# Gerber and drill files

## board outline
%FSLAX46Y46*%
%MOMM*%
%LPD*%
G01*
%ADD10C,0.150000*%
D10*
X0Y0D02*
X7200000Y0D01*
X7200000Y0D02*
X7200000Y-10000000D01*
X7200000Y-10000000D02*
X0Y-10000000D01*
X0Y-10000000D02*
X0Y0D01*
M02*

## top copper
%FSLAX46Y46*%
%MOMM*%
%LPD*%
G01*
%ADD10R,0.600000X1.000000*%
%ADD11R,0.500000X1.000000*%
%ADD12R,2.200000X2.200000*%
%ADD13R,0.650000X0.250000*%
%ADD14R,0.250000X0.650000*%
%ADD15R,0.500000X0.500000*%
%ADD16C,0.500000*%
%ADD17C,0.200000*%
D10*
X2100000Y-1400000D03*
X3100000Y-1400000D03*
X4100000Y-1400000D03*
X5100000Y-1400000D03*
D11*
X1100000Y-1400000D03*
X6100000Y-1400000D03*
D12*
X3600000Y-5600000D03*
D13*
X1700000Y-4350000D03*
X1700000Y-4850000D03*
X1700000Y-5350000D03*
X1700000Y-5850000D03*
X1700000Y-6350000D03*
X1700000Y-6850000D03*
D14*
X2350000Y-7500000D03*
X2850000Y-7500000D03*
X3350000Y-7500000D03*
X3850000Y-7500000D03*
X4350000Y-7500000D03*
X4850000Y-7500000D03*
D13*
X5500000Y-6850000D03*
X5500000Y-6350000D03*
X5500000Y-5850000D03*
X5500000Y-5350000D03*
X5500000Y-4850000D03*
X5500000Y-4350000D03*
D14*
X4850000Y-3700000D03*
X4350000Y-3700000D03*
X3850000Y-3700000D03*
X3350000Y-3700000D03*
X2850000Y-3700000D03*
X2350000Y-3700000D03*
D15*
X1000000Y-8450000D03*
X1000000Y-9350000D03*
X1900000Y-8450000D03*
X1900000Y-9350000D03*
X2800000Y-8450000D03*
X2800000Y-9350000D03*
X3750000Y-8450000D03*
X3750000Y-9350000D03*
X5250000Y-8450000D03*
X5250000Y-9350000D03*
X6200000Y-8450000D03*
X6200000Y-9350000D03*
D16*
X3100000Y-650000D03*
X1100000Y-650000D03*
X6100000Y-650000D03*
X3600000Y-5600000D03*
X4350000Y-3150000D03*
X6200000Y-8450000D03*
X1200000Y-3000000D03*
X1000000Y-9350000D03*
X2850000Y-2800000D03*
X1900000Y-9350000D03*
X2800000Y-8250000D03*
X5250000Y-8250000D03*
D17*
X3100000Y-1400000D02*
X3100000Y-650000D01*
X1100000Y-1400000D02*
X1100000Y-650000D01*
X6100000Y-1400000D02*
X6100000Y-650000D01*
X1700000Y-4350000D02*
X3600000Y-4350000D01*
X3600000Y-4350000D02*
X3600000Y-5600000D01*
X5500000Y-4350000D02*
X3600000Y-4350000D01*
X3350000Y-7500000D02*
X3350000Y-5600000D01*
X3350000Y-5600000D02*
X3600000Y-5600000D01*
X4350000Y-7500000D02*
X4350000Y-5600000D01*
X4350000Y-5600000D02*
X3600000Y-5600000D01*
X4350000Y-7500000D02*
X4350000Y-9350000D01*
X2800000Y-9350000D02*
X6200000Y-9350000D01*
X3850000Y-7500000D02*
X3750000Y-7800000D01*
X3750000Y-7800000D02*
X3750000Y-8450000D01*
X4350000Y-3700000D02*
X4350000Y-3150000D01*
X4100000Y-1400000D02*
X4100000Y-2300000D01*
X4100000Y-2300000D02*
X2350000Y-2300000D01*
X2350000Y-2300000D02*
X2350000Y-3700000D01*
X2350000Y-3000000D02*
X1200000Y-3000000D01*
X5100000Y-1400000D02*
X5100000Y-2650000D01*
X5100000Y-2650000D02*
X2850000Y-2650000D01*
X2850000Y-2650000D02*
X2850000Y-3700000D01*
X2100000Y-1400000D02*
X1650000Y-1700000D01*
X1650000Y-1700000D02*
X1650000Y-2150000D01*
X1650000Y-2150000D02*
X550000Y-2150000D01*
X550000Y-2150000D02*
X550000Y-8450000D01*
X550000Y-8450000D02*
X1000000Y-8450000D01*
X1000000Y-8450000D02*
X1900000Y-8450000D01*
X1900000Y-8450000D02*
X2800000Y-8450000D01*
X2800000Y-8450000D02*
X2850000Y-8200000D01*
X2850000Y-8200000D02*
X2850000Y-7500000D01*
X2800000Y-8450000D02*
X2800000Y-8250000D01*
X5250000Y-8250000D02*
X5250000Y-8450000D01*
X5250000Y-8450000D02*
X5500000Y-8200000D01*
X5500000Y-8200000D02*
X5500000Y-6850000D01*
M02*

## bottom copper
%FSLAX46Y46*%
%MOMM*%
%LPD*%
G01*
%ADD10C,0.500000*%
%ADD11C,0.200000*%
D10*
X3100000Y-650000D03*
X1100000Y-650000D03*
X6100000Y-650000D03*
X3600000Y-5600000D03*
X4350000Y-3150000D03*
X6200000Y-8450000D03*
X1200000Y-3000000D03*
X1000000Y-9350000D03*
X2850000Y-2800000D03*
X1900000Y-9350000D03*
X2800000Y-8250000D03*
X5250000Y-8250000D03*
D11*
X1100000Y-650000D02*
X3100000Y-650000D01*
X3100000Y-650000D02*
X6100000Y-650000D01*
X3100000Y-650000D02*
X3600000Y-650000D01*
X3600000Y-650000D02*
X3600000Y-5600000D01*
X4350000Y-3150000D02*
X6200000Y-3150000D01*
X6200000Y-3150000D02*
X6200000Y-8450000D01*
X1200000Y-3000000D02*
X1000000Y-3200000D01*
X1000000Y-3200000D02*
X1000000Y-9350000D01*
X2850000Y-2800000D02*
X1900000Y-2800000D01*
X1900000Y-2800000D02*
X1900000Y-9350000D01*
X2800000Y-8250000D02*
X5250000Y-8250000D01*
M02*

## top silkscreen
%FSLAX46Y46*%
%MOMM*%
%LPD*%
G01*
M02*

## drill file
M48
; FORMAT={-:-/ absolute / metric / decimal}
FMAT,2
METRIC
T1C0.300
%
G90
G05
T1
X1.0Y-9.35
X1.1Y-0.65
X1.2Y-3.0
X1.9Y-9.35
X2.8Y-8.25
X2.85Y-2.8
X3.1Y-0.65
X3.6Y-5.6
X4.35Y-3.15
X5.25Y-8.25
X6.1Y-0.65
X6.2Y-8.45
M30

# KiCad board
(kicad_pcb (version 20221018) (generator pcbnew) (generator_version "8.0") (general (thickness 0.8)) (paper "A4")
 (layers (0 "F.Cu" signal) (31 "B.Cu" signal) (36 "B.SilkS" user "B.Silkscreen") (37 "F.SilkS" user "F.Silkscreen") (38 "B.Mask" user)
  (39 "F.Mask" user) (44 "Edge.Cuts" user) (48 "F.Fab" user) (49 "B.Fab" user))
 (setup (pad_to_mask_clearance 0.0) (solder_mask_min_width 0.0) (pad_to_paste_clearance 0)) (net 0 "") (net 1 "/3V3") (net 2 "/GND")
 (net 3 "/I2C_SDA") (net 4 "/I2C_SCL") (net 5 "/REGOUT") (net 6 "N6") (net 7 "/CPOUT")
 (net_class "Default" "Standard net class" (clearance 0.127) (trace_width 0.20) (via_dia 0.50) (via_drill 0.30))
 (gr_line (start 0 0) (end 7.2 0) (layer "Edge.Cuts") (width 0.15))
 (gr_line (start 7.2 0) (end 7.2 10.0) (layer "Edge.Cuts") (width 0.15))
 (gr_line (start 7.2 10.0) (end 0 10.0) (layer "Edge.Cuts") (width 0.15))
 (gr_line (start 0 10.0) (end 0 0) (layer "Edge.Cuts") (width 0.15))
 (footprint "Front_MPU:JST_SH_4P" (layer "F.Cu") (at 3.6 1.4)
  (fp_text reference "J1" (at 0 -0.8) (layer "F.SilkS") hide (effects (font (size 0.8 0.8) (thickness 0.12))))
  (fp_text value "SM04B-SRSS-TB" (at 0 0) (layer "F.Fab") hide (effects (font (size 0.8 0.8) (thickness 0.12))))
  (pad "1" smd rect (at -1.5 0) (size 0.6 1.0) (layers "F.Cu" "F.Paste" "F.Mask") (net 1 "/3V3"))
  (pad "2" smd rect (at -0.5 0) (size 0.6 1.0) (layers "F.Cu" "F.Paste" "F.Mask") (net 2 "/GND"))
  (pad "3" smd rect (at 0.5 0) (size 0.6 1.0) (layers "F.Cu" "F.Paste" "F.Mask") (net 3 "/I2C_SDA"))
  (pad "4" smd rect (at 1.5 0) (size 0.6 1.0) (layers "F.Cu" "F.Paste" "F.Mask") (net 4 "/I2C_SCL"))
  (pad "5" smd rect (at -2.5 0) (size 0.5 1.0) (layers "F.Cu" "F.Paste" "F.Mask") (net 2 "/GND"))
  (pad "5" smd rect (at 2.5 0) (size 0.5 1.0) (layers "F.Cu" "F.Paste" "F.Mask") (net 2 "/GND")))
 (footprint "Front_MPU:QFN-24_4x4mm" (layer "F.Cu") (at 3.6 5.6)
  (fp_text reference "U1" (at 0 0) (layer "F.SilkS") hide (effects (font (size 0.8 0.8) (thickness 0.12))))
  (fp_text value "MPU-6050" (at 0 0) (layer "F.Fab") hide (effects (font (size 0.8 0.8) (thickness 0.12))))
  (pad "25" smd rect (at 0 0) (size 2.2 2.2) (layers "F.Cu" "F.Paste" "F.Mask") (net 2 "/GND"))
  (pad "1" smd rect (at -1.90 -1.25) (size 0.65 0.25) (layers "F.Cu" "F.Paste" "F.Mask") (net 2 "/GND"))
  (pad "2" smd rect (at -1.90 -0.75) (size 0.65 0.25) (layers "F.Cu" "F.Paste" "F.Mask") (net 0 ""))
  (pad "3" smd rect (at -1.90 -0.25) (size 0.65 0.25) (layers "F.Cu" "F.Paste" "F.Mask") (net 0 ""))
  (pad "4" smd rect (at -1.90 0.25) (size 0.65 0.25) (layers "F.Cu" "F.Paste" "F.Mask") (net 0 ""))
  (pad "5" smd rect (at -1.90 0.75) (size 0.65 0.25) (layers "F.Cu" "F.Paste" "F.Mask") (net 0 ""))
  (pad "6" smd rect (at -1.90 1.25) (size 0.65 0.25) (layers "F.Cu" "F.Paste" "F.Mask") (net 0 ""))
  (pad "7" smd rect (at -1.25 1.90) (size 0.25 0.65) (layers "F.Cu" "F.Paste" "F.Mask") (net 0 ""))
  (pad "8" smd rect (at -0.75 1.90) (size 0.25 0.65) (layers "F.Cu" "F.Paste" "F.Mask") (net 1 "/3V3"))
  (pad "9" smd rect (at -0.25 1.90) (size 0.25 0.65) (layers "F.Cu" "F.Paste" "F.Mask") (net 2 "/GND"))
  (pad "10" smd rect (at 0.25 1.90) (size 0.25 0.65) (layers "F.Cu" "F.Paste" "F.Mask") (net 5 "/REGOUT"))
  (pad "11" smd rect (at 0.75 1.90) (size 0.25 0.65) (layers "F.Cu" "F.Paste" "F.Mask") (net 2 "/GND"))
  (pad "12" smd rect (at 1.25 1.90) (size 0.25 0.65) (layers "F.Cu" "F.Paste" "F.Mask") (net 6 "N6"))
  (pad "13" smd rect (at 1.90 1.25) (size 0.65 0.25) (layers "F.Cu" "F.Paste" "F.Mask") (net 1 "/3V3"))
  (pad "14" smd rect (at 1.90 0.75) (size 0.65 0.25) (layers "F.Cu" "F.Paste" "F.Mask") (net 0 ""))
  (pad "15" smd rect (at 1.90 0.25) (size 0.65 0.25) (layers "F.Cu" "F.Paste" "F.Mask") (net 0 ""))
  (pad "16" smd rect (at 1.90 -0.25) (size 0.65 0.25) (layers "F.Cu" "F.Paste" "F.Mask") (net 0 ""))
  (pad "17" smd rect (at 1.90 -0.75) (size 0.65 0.25) (layers "F.Cu" "F.Paste" "F.Mask") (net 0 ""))
  (pad "18" smd rect (at 1.90 -1.25) (size 0.65 0.25) (layers "F.Cu" "F.Paste" "F.Mask") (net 2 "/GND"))
  (pad "19" smd rect (at 1.25 -1.90) (size 0.25 0.65) (layers "F.Cu" "F.Paste" "F.Mask") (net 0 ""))
  (pad "20" smd rect (at 0.75 -1.90) (size 0.25 0.65) (layers "F.Cu" "F.Paste" "F.Mask") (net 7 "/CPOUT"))
  (pad "21" smd rect (at 0.25 -1.90) (size 0.25 0.65) (layers "F.Cu" "F.Paste" "F.Mask") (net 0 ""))
  (pad "22" smd rect (at -0.25 -1.90) (size 0.25 0.65) (layers "F.Cu" "F.Paste" "F.Mask") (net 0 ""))
  (pad "23" smd rect (at -0.75 -1.90) (size 0.25 0.65) (layers "F.Cu" "F.Paste" "F.Mask") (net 4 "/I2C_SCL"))
  (pad "24" smd rect (at -1.25 -1.90) (size 0.25 0.65) (layers "F.Cu" "F.Paste" "F.Mask") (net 3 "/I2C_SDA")))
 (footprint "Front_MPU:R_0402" (layer "F.Cu") (at 1.00 8.90)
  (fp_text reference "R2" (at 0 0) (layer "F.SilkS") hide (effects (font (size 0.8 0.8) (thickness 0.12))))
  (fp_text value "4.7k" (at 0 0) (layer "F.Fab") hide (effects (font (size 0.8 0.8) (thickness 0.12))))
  (pad "1" smd rect (at 0 -0.45) (size 0.5 0.5) (layers "F.Cu" "F.Paste" "F.Mask") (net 1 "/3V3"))
  (pad "2" smd rect (at 0 0.45) (size 0.5 0.5) (layers "F.Cu" "F.Paste" "F.Mask") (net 3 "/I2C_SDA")))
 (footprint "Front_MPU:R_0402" (layer "F.Cu") (at 1.90 8.90)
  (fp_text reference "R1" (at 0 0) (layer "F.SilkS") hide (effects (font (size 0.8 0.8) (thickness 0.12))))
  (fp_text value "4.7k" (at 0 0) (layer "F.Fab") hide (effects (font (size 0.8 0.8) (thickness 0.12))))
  (pad "1" smd rect (at 0 -0.45) (size 0.5 0.5) (layers "F.Cu" "F.Paste" "F.Mask") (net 1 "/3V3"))
  (pad "2" smd rect (at 0 0.45) (size 0.5 0.5) (layers "F.Cu" "F.Paste" "F.Mask") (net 4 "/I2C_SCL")))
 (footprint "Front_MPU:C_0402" (layer "F.Cu") (at 2.80 8.90)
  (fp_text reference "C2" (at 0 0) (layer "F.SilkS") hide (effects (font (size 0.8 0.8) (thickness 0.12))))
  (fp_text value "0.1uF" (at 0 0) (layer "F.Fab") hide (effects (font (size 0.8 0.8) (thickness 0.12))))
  (pad "1" smd rect (at 0 -0.45) (size 0.5 0.5) (layers "F.Cu" "F.Paste" "F.Mask") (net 1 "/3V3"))
  (pad "2" smd rect (at 0 0.45) (size 0.5 0.5) (layers "F.Cu" "F.Paste" "F.Mask") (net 2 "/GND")))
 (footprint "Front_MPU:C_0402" (layer "F.Cu") (at 3.75 8.90)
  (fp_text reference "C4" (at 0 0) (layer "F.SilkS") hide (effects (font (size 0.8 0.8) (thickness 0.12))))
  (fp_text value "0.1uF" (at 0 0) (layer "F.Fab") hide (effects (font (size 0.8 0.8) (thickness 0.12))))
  (pad "1" smd rect (at 0 -0.45) (size 0.5 0.5) (layers "F.Cu" "F.Paste" "F.Mask") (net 5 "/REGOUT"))
  (pad "2" smd rect (at 0 0.45) (size 0.5 0.5) (layers "F.Cu" "F.Paste" "F.Mask") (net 2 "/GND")))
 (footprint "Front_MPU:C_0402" (layer "F.Cu") (at 5.25 8.90)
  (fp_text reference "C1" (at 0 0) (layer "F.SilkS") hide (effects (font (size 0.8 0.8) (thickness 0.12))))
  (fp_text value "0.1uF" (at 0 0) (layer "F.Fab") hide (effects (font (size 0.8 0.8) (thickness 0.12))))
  (pad "1" smd rect (at 0 -0.45) (size 0.5 0.5) (layers "F.Cu" "F.Paste" "F.Mask") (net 1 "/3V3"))
  (pad "2" smd rect (at 0 0.45) (size 0.5 0.5) (layers "F.Cu" "F.Paste" "F.Mask") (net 2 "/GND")))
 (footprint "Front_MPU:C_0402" (layer "F.Cu") (at 6.20 8.90)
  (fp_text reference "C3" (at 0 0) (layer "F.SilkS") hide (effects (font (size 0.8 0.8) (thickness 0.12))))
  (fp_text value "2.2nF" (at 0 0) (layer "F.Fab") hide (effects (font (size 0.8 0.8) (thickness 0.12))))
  (pad "1" smd rect (at 0 -0.45) (size 0.5 0.5) (layers "F.Cu" "F.Paste" "F.Mask") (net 7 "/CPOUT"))
  (pad "2" smd rect (at 0 0.45) (size 0.5 0.5) (layers "F.Cu" "F.Paste" "F.Mask") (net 2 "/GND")))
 (segment (start 3.10 1.40) (end 3.10 0.65) (width 0.20) (layer "F.Cu") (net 2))
 (via (at 3.10 0.65) (size 0.50) (drill 0.30) (layers "F.Cu" "B.Cu") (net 2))
 (segment (start 1.10 1.40) (end 1.10 0.65) (width 0.20) (layer "F.Cu") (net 2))
 (via (at 1.10 0.65) (size 0.50) (drill 0.30) (layers "F.Cu" "B.Cu") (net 2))
 (segment (start 6.10 1.40) (end 6.10 0.65) (width 0.20) (layer "F.Cu") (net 2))
 (via (at 6.10 0.65) (size 0.50) (drill 0.30) (layers "F.Cu" "B.Cu") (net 2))
 (segment (start 1.10 0.65) (end 3.10 0.65) (width 0.20) (layer "B.Cu") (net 2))
 (segment (start 3.10 0.65) (end 6.10 0.65) (width 0.20) (layer "B.Cu") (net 2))
 (segment (start 3.10 0.65) (end 3.60 0.65) (width 0.20) (layer "B.Cu") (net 2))
 (segment (start 3.60 0.65) (end 3.60 5.60) (width 0.20) (layer "B.Cu") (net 2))
 (via (at 3.60 5.60) (size 0.50) (drill 0.30) (layers "F.Cu" "B.Cu") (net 2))
 (segment (start 1.70 4.35) (end 3.60 4.35) (width 0.20) (layer "F.Cu") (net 2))
 (segment (start 3.60 4.35) (end 3.60 5.60) (width 0.20) (layer "F.Cu") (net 2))
 (segment (start 5.50 4.35) (end 3.60 4.35) (width 0.20) (layer "F.Cu") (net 2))
 (segment (start 3.35 7.50) (end 3.35 5.60) (width 0.20) (layer "F.Cu") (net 2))
 (segment (start 3.35 5.60) (end 3.60 5.60) (width 0.20) (layer "F.Cu") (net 2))
 (segment (start 4.35 7.50) (end 4.35 5.60) (width 0.20) (layer "F.Cu") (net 2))
 (segment (start 4.35 5.60) (end 3.60 5.60) (width 0.20) (layer "F.Cu") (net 2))
 (segment (start 4.35 7.50) (end 4.35 9.35) (width 0.20) (layer "F.Cu") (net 2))
 (segment (start 2.80 9.35) (end 6.20 9.35) (width 0.20) (layer "F.Cu") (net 2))
 (segment (start 3.85 7.50) (end 3.75 7.80) (width 0.20) (layer "F.Cu") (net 5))
 (segment (start 3.75 7.80) (end 3.75 8.45) (width 0.20) (layer "F.Cu") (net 5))
 (segment (start 4.35 3.70) (end 4.35 3.15) (width 0.20) (layer "F.Cu") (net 7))
 (via (at 4.35 3.15) (size 0.50) (drill 0.30) (layers "F.Cu" "B.Cu") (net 7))
 (segment (start 4.35 3.15) (end 6.20 3.15) (width 0.20) (layer "B.Cu") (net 7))
 (segment (start 6.20 3.15) (end 6.20 8.45) (width 0.20) (layer "B.Cu") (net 7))
 (via (at 6.20 8.45) (size 0.50) (drill 0.30) (layers "F.Cu" "B.Cu") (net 7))
 (segment (start 4.10 1.40) (end 4.10 2.30) (width 0.20) (layer "F.Cu") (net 3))
 (segment (start 4.10 2.30) (end 2.35 2.30) (width 0.20) (layer "F.Cu") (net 3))
 (segment (start 2.35 2.30) (end 2.35 3.70) (width 0.20) (layer "F.Cu") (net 3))
 (segment (start 2.35 3.00) (end 1.20 3.00) (width 0.20) (layer "F.Cu") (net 3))
 (via (at 1.20 3.00) (size 0.50) (drill 0.30) (layers "F.Cu" "B.Cu") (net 3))
 (segment (start 1.20 3.00) (end 1.00 3.20) (width 0.20) (layer "B.Cu") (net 3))
 (segment (start 1.00 3.20) (end 1.00 9.35) (width 0.20) (layer "B.Cu") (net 3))
 (via (at 1.00 9.35) (size 0.50) (drill 0.30) (layers "F.Cu" "B.Cu") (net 3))
 (segment (start 5.10 1.40) (end 5.10 2.65) (width 0.20) (layer "F.Cu") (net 4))
 (segment (start 5.10 2.65) (end 2.85 2.65) (width 0.20) (layer "F.Cu") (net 4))
 (segment (start 2.85 2.65) (end 2.85 3.70) (width 0.20) (layer "F.Cu") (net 4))
 (via (at 2.85 2.80) (size 0.50) (drill 0.30) (layers "F.Cu" "B.Cu") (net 4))
 (segment (start 2.85 2.80) (end 1.90 2.80) (width 0.20) (layer "B.Cu") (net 4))
 (segment (start 1.90 2.80) (end 1.90 9.35) (width 0.20) (layer "B.Cu") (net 4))
 (via (at 1.90 9.35) (size 0.50) (drill 0.30) (layers "F.Cu" "B.Cu") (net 4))
 (segment (start 2.10 1.40) (end 1.65 1.70) (width 0.20) (layer "F.Cu") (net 1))
 (segment (start 1.65 1.70) (end 1.65 2.15) (width 0.20) (layer "F.Cu") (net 1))
 (segment (start 1.65 2.15) (end 0.55 2.15) (width 0.20) (layer "F.Cu") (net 1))
 (segment (start 0.55 2.15) (end 0.55 8.45) (width 0.20) (layer "F.Cu") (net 1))
 (segment (start 0.55 8.45) (end 1.00 8.45) (width 0.20) (layer "F.Cu") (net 1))
 (segment (start 1.00 8.45) (end 1.90 8.45) (width 0.20) (layer "F.Cu") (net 1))
 (segment (start 1.90 8.45) (end 2.80 8.45) (width 0.20) (layer "F.Cu") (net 1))
 (segment (start 2.80 8.45) (end 2.85 8.20) (width 0.20) (layer "F.Cu") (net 1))
 (segment (start 2.85 8.20) (end 2.85 7.50) (width 0.20) (layer "F.Cu") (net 1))
 (segment (start 2.80 8.45) (end 2.80 8.25) (width 0.20) (layer "F.Cu") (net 1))
 (via (at 2.80 8.25) (size 0.50) (drill 0.30) (layers "F.Cu" "B.Cu") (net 1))
 (segment (start 2.80 8.25) (end 5.25 8.25) (width 0.20) (layer "B.Cu") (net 1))
 (via (at 5.25 8.25) (size 0.50) (drill 0.30) (layers "F.Cu" "B.Cu") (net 1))
 (segment (start 5.25 8.25) (end 5.25 8.45) (width 0.20) (layer "F.Cu") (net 1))
 (segment (start 5.25 8.45) (end 5.50 8.20) (width 0.20) (layer "F.Cu") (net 1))
 (segment (start 5.50 8.20) (end 5.50 6.85) (width 0.20) (layer "F.Cu") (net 1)))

